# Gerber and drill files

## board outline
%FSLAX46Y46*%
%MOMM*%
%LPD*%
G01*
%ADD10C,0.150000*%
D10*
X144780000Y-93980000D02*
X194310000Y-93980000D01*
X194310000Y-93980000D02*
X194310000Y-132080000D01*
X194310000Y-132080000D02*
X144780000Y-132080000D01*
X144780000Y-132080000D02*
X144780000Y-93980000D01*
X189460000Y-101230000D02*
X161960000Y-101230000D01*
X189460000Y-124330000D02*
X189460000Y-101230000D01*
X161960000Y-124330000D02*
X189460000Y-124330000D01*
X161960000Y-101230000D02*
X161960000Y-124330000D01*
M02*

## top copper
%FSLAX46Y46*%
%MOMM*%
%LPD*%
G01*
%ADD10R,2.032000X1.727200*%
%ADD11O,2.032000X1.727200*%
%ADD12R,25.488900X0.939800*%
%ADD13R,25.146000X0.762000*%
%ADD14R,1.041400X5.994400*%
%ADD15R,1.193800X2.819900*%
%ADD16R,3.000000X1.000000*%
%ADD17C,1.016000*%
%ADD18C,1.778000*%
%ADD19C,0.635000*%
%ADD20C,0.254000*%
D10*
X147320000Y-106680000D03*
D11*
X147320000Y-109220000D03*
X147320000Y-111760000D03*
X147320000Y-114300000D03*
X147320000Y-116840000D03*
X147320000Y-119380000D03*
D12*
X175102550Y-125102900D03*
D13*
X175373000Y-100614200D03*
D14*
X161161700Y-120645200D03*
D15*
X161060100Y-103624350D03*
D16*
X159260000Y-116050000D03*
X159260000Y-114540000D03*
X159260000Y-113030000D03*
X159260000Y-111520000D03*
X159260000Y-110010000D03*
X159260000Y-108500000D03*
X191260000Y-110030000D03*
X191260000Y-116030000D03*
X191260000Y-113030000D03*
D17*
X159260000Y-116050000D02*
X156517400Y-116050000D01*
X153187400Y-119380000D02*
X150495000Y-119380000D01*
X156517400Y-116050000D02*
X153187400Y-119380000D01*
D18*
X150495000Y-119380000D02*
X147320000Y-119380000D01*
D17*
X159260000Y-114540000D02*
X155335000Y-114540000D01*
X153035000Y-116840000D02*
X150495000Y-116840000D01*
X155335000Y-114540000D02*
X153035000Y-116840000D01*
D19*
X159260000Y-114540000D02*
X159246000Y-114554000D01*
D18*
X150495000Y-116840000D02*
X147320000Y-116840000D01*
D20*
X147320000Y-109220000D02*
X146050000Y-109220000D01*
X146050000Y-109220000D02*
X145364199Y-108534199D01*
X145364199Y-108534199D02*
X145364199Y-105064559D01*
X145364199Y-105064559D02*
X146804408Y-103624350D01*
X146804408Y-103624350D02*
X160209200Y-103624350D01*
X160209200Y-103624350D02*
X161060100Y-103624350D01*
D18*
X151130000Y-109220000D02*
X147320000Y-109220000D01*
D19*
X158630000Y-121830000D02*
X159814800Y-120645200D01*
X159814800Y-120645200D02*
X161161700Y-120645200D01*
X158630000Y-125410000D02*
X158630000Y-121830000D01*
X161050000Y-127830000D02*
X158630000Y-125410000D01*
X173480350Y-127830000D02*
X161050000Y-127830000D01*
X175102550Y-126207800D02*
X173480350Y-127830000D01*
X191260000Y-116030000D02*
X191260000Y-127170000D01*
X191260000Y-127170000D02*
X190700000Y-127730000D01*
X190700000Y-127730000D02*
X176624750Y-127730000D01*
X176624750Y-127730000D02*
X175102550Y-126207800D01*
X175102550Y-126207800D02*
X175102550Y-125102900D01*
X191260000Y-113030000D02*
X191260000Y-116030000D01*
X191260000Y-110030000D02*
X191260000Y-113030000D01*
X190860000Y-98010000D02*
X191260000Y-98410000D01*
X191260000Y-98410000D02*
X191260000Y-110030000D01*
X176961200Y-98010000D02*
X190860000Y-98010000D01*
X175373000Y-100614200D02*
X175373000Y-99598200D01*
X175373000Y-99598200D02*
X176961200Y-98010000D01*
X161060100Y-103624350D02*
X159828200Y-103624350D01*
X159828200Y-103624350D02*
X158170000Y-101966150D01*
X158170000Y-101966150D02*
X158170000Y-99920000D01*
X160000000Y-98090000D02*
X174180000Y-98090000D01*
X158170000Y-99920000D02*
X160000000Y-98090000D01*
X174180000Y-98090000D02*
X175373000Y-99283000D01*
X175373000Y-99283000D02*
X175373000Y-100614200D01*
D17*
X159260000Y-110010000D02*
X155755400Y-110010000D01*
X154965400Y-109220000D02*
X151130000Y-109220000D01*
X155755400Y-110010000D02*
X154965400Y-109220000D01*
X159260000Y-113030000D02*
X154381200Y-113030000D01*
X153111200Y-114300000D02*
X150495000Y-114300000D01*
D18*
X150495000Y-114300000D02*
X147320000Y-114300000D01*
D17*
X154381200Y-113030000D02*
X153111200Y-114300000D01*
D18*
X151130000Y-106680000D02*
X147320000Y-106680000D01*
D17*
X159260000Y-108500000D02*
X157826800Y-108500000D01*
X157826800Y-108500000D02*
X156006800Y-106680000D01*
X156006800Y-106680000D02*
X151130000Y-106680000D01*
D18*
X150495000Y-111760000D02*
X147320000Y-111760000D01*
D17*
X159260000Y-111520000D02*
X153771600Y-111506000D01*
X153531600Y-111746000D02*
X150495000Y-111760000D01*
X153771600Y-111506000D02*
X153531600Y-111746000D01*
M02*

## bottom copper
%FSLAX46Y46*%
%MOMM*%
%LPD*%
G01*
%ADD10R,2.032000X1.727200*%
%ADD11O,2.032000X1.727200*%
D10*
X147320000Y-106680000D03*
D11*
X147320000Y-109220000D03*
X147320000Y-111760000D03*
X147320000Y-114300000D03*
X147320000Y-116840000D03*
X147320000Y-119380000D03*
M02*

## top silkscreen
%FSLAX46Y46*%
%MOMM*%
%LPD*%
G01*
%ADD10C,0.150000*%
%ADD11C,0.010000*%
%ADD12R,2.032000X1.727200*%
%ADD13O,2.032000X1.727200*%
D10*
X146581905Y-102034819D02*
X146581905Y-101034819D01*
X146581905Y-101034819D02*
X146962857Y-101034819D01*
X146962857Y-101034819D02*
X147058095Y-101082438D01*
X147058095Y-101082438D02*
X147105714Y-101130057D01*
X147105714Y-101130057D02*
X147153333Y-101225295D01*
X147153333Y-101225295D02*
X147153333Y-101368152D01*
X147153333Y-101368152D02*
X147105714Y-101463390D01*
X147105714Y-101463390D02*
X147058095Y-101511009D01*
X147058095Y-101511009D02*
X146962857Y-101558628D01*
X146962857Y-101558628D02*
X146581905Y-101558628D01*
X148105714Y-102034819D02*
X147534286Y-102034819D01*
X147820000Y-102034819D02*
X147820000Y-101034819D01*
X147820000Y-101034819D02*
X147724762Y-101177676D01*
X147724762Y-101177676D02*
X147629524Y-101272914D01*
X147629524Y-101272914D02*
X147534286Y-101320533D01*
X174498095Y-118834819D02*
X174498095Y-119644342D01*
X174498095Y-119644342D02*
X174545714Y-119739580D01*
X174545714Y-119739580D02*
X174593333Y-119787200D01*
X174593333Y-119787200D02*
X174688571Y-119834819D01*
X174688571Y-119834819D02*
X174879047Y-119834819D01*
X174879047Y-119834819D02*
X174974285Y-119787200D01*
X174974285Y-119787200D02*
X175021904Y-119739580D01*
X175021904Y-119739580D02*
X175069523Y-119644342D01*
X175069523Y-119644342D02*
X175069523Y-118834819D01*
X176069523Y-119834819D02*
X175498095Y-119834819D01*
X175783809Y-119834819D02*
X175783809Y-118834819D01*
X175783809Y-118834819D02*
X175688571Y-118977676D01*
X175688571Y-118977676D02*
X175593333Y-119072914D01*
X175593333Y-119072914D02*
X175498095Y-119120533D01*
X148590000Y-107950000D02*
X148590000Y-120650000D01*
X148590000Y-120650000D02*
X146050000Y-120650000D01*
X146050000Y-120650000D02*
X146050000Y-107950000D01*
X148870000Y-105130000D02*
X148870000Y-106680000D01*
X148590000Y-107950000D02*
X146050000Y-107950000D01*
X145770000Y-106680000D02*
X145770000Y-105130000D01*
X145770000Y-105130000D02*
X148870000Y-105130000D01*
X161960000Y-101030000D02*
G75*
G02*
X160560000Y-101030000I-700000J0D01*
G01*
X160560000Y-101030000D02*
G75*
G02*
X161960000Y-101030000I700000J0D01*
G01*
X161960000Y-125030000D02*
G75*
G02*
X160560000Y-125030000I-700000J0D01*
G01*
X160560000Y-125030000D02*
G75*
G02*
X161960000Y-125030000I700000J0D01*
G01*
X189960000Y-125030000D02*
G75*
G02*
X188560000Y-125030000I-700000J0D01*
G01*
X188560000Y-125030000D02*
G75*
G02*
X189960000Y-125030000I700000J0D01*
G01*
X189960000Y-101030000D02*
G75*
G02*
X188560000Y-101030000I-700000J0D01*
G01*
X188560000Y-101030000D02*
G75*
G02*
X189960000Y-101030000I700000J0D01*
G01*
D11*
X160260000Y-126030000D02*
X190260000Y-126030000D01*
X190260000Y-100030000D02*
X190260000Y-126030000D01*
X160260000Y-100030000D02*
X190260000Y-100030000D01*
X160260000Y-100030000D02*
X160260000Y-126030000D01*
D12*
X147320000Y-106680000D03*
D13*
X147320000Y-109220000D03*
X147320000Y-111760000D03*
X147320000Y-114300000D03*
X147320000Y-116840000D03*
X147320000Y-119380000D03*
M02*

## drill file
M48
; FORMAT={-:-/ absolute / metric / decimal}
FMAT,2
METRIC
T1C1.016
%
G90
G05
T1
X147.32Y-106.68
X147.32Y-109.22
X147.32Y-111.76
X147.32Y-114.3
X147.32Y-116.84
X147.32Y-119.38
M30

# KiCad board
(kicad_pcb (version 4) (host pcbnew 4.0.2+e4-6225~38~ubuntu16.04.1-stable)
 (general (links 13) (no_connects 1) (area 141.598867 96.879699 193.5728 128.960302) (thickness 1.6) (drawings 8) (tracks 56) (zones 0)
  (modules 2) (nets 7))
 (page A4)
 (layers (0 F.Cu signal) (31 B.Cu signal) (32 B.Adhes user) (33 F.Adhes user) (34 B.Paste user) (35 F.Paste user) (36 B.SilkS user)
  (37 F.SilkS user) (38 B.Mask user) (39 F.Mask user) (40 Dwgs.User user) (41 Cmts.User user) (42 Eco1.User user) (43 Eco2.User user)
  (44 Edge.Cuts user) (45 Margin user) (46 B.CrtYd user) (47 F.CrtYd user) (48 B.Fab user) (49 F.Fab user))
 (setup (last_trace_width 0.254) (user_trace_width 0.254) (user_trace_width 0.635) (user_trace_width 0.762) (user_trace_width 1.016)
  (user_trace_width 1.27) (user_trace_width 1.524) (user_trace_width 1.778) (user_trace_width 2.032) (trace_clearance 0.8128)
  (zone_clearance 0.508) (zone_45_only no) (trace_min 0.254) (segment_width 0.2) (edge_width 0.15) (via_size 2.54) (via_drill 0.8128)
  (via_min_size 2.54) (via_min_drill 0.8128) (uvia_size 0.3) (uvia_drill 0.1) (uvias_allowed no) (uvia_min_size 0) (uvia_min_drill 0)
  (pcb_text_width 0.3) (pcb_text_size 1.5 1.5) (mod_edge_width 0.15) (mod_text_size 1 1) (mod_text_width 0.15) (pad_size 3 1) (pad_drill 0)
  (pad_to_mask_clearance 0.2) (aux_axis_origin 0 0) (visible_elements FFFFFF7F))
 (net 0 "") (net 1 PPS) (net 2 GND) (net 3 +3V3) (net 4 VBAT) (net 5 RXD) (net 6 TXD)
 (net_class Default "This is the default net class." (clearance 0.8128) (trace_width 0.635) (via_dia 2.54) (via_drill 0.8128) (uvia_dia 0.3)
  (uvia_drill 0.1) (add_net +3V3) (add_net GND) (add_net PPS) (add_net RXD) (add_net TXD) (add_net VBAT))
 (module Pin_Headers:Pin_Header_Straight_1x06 (layer F.Cu) (at 147.32 106.68)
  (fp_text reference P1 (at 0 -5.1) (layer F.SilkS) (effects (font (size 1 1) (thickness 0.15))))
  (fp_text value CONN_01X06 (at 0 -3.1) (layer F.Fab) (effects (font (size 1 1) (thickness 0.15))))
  (fp_line (start 1.27 1.27) (end 1.27 13.97) (layer F.SilkS) (width 0.15))
  (fp_line (start 1.27 13.97) (end -1.27 13.97) (layer F.SilkS) (width 0.15))
  (fp_line (start -1.27 13.97) (end -1.27 1.27) (layer F.SilkS) (width 0.15))
  (fp_line (start 1.55 -1.55) (end 1.55 0) (layer F.SilkS) (width 0.15))
  (fp_line (start 1.27 1.27) (end -1.27 1.27) (layer F.SilkS) (width 0.15))
  (fp_line (start -1.55 0) (end -1.55 -1.55) (layer F.SilkS) (width 0.15))
  (fp_line (start -1.55 -1.55) (end 1.55 -1.55) (layer F.SilkS) (width 0.15))
  (pad 1 thru_hole rect (at 0 0) (size 2.032 1.7272) (drill 1.016) (layers *.Cu *.Mask F.SilkS) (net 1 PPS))
  (pad 2 thru_hole oval (at 0 2.54) (size 2.032 1.7272) (drill 1.016) (layers *.Cu *.Mask F.SilkS) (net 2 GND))
  (pad 3 thru_hole oval (at 0 5.08) (size 2.032 1.7272) (drill 1.016) (layers *.Cu *.Mask F.SilkS) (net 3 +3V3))
  (pad 4 thru_hole oval (at 0 7.62) (size 2.032 1.7272) (drill 1.016) (layers *.Cu *.Mask F.SilkS) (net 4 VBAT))
  (pad 5 thru_hole oval (at 0 10.16) (size 2.032 1.7272) (drill 1.016) (layers *.Cu *.Mask F.SilkS) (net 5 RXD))
  (pad 6 thru_hole oval (at 0 12.7) (size 2.032 1.7272) (drill 1.016) (layers *.Cu *.Mask F.SilkS) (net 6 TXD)))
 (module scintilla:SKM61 (layer F.Cu) (at 175.26 113.03)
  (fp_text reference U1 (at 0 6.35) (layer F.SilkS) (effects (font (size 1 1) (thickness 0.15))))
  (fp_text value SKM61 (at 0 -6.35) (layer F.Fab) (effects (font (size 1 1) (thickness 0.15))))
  (fp_circle (center -14 -12) (end -14.7 -12) (layer F.SilkS) (width 0.15))
  (fp_circle (center -14 12) (end -13.3 12) (layer F.SilkS) (width 0.15))
  (fp_circle (center 14 12) (end 14 11.3) (layer F.SilkS) (width 0.15))
  (fp_circle (center 14 -12) (end 14.7 -12) (layer F.SilkS) (width 0.15))
  (fp_line (start -15 13) (end 15 13) (layer F.SilkS) (width 0.01))
  (fp_line (start 15 -13) (end 15 13) (layer F.SilkS) (width 0.01))
  (fp_line (start -15 -13) (end 15 -13) (layer F.SilkS) (width 0.01))
  (fp_line (start -15 -13) (end -15 13) (layer F.SilkS) (width 0.01))
  (pad 7 smd rect (at -0.15745 12.0729) (size 25.4889 0.9398) (layers F.Cu F.Paste F.Mask) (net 2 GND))
  (pad 8 smd rect (at 0.113 -12.4158) (size 25.146 0.762) (layers F.Cu F.Paste F.Mask) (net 2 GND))
  (pad 9 smd rect (at -14.0983 7.6152) (size 1.0414 5.9944) (layers F.Cu F.Paste F.Mask) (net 2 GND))
  (pad 10 smd rect (at -14.1999 -9.40565) (size 1.1938 2.8199) (layers F.Cu F.Paste F.Mask) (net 2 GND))
  (pad 1 smd rect (at -16 3.02) (size 3 1) (layers F.Cu F.Paste F.Mask) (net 6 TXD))
  (pad 2 smd rect (at -16 1.51) (size 3 1) (layers F.Cu F.Paste F.Mask) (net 5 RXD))
  (pad 3 smd rect (at -16 0) (size 3 1) (layers F.Cu F.Paste F.Mask) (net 4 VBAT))
  (pad 4 smd rect (at -16 -1.51) (size 3 1) (layers F.Cu F.Paste F.Mask) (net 3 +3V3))
  (pad 5 smd rect (at -16 -3.02) (size 3 1) (layers F.Cu F.Paste F.Mask) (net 2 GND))
  (pad 6 smd rect (at -16 -4.53) (size 3 1) (layers F.Cu F.Paste F.Mask) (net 1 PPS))
  (pad 11 smd rect (at 16 -3) (size 3 1) (layers F.Cu F.Paste F.Mask) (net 2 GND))
  (pad 13 smd rect (at 16 3) (size 3 1) (layers F.Cu F.Paste F.Mask) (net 2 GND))
  (pad 12 smd rect (at 16 0) (size 3 1) (layers F.Cu F.Paste F.Mask) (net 2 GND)))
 (gr_line (start 144.78 93.98) (end 194.31 93.98) (angle 90) (layer Edge.Cuts) (width 0.15))
 (gr_line (start 194.31 93.98) (end 194.31 132.08) (angle 90) (layer Edge.Cuts) (width 0.15))
 (gr_line (start 194.31 132.08) (end 144.78 132.08) (angle 90) (layer Edge.Cuts) (width 0.15))
 (gr_line (start 144.78 132.08) (end 144.78 93.98) (angle 90) (layer Edge.Cuts) (width 0.15))
 (gr_line (start 189.46 101.23) (end 161.96 101.23) (angle 90) (layer Edge.Cuts) (width 0.15))
 (gr_line (start 189.46 124.33) (end 189.46 101.23) (angle 90) (layer Edge.Cuts) (width 0.15))
 (gr_line (start 161.96 124.33) (end 189.46 124.33) (angle 90) (layer Edge.Cuts) (width 0.15))
 (gr_line (start 161.96 101.23) (end 161.96 124.33) (angle 90) (layer Edge.Cuts) (width 0.15))
 (segment (start 159.26 116.05) (end 156.5174 116.05) (width 1.016) (layer F.Cu) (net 6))
 (segment (start 153.1874 119.38) (end 150.495 119.38) (width 1.016) (layer F.Cu) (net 6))
 (segment (start 156.5174 116.05) (end 153.1874 119.38) (width 1.016) (layer F.Cu) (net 6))
 (segment (start 150.495 119.38) (end 147.32 119.38) (width 1.778) (layer F.Cu) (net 6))
 (segment (start 159.26 114.54) (end 155.335 114.54) (width 1.016) (layer F.Cu) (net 5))
 (segment (start 153.035 116.84) (end 150.495 116.84) (width 1.016) (layer F.Cu) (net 5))
 (segment (start 155.335 114.54) (end 153.035 116.84) (width 1.016) (layer F.Cu) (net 5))
 (segment (start 159.26 114.54) (end 159.246 114.554) (width 0.635) (layer F.Cu) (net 5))
 (segment (start 150.495 116.84) (end 147.32 116.84) (width 1.778) (layer F.Cu) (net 5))
 (segment (start 147.32 109.22) (end 146.05 109.22) (width 0.254) (layer F.Cu) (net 2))
 (segment (start 146.05 109.22) (end 145.364199 108.534199) (width 0.254) (layer F.Cu) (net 2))
 (segment (start 145.364199 108.534199) (end 145.364199 105.064559) (width 0.254) (layer F.Cu) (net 2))
 (segment (start 145.364199 105.064559) (end 146.804408 103.62435) (width 0.254) (layer F.Cu) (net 2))
 (segment (start 146.804408 103.62435) (end 160.2092 103.62435) (width 0.254) (layer F.Cu) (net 2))
 (segment (start 160.2092 103.62435) (end 161.0601 103.62435) (width 0.254) (layer F.Cu) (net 2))
 (segment (start 151.13 109.22) (end 147.32 109.22) (width 1.778) (layer F.Cu) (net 2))
 (segment (start 158.63 121.83) (end 159.8148 120.6452) (width 0.635) (layer F.Cu) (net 2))
 (segment (start 159.8148 120.6452) (end 161.1617 120.6452) (width 0.635) (layer F.Cu) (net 2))
 (segment (start 158.63 125.41) (end 158.63 121.83) (width 0.635) (layer F.Cu) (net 2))
 (segment (start 161.05 127.83) (end 158.63 125.41) (width 0.635) (layer F.Cu) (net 2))
 (segment (start 173.48035 127.83) (end 161.05 127.83) (width 0.635) (layer F.Cu) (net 2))
 (segment (start 175.10255 126.2078) (end 173.48035 127.83) (width 0.635) (layer F.Cu) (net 2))
 (segment (start 191.26 116.03) (end 191.26 127.17) (width 0.635) (layer F.Cu) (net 2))
 (segment (start 191.26 127.17) (end 190.7 127.73) (width 0.635) (layer F.Cu) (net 2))
 (segment (start 190.7 127.73) (end 176.62475 127.73) (width 0.635) (layer F.Cu) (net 2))
 (segment (start 176.62475 127.73) (end 175.10255 126.2078) (width 0.635) (layer F.Cu) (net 2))
 (segment (start 175.10255 126.2078) (end 175.10255 125.1029) (width 0.635) (layer F.Cu) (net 2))
 (segment (start 191.26 113.03) (end 191.26 116.03) (width 0.635) (layer F.Cu) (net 2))
 (segment (start 191.26 110.03) (end 191.26 113.03) (width 0.635) (layer F.Cu) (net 2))
 (segment (start 190.86 98.01) (end 191.26 98.41) (width 0.635) (layer F.Cu) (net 2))
 (segment (start 191.26 98.41) (end 191.26 110.03) (width 0.635) (layer F.Cu) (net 2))
 (segment (start 176.9612 98.01) (end 190.86 98.01) (width 0.635) (layer F.Cu) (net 2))
 (segment (start 175.373 100.6142) (end 175.373 99.5982) (width 0.635) (layer F.Cu) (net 2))
 (segment (start 175.373 99.5982) (end 176.9612 98.01) (width 0.635) (layer F.Cu) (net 2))
 (segment (start 161.0601 103.62435) (end 159.8282 103.62435) (width 0.635) (layer F.Cu) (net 2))
 (segment (start 159.8282 103.62435) (end 158.17 101.96615) (width 0.635) (layer F.Cu) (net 2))
 (segment (start 158.17 101.96615) (end 158.17 99.92) (width 0.635) (layer F.Cu) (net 2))
 (segment (start 160 98.09) (end 174.18 98.09) (width 0.635) (layer F.Cu) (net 2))
 (segment (start 158.17 99.92) (end 160 98.09) (width 0.635) (layer F.Cu) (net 2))
 (segment (start 174.18 98.09) (end 175.373 99.283) (width 0.635) (layer F.Cu) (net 2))
 (segment (start 175.373 99.283) (end 175.373 100.6142) (width 0.635) (layer F.Cu) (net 2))
 (segment (start 159.26 110.01) (end 155.7554 110.01) (width 1.016) (layer F.Cu) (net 2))
 (segment (start 154.9654 109.22) (end 151.13 109.22) (width 1.016) (layer F.Cu) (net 2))
 (segment (start 155.7554 110.01) (end 154.9654 109.22) (width 1.016) (layer F.Cu) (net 2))
 (segment (start 159.26 113.03) (end 154.3812 113.03) (width 1.016) (layer F.Cu) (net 4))
 (segment (start 153.1112 114.3) (end 150.495 114.3) (width 1.016) (layer F.Cu) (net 4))
 (segment (start 150.495 114.3) (end 147.32 114.3) (width 1.778) (layer F.Cu) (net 4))
 (segment (start 154.3812 113.03) (end 153.1112 114.3) (width 1.016) (layer F.Cu) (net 4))
 (segment (start 151.13 106.68) (end 147.32 106.68) (width 1.778) (layer F.Cu) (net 1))
 (segment (start 159.26 108.5) (end 157.8268 108.5) (width 1.016) (layer F.Cu) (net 1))
 (segment (start 157.8268 108.5) (end 156.0068 106.68) (width 1.016) (layer F.Cu) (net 1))
 (segment (start 156.0068 106.68) (end 151.13 106.68) (width 1.016) (layer F.Cu) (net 1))
 (segment (start 150.495 111.76) (end 147.32 111.76) (width 1.778) (layer F.Cu) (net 3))
 (segment (start 159.26 111.52) (end 153.7716 111.506) (width 1.016) (layer F.Cu) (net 3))
 (segment (start 153.5316 111.746) (end 150.495 111.76) (width 1.016) (layer F.Cu) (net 3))
 (segment (start 153.7716 111.506) (end 153.5316 111.746) (width 1.016) (layer F.Cu) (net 3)))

